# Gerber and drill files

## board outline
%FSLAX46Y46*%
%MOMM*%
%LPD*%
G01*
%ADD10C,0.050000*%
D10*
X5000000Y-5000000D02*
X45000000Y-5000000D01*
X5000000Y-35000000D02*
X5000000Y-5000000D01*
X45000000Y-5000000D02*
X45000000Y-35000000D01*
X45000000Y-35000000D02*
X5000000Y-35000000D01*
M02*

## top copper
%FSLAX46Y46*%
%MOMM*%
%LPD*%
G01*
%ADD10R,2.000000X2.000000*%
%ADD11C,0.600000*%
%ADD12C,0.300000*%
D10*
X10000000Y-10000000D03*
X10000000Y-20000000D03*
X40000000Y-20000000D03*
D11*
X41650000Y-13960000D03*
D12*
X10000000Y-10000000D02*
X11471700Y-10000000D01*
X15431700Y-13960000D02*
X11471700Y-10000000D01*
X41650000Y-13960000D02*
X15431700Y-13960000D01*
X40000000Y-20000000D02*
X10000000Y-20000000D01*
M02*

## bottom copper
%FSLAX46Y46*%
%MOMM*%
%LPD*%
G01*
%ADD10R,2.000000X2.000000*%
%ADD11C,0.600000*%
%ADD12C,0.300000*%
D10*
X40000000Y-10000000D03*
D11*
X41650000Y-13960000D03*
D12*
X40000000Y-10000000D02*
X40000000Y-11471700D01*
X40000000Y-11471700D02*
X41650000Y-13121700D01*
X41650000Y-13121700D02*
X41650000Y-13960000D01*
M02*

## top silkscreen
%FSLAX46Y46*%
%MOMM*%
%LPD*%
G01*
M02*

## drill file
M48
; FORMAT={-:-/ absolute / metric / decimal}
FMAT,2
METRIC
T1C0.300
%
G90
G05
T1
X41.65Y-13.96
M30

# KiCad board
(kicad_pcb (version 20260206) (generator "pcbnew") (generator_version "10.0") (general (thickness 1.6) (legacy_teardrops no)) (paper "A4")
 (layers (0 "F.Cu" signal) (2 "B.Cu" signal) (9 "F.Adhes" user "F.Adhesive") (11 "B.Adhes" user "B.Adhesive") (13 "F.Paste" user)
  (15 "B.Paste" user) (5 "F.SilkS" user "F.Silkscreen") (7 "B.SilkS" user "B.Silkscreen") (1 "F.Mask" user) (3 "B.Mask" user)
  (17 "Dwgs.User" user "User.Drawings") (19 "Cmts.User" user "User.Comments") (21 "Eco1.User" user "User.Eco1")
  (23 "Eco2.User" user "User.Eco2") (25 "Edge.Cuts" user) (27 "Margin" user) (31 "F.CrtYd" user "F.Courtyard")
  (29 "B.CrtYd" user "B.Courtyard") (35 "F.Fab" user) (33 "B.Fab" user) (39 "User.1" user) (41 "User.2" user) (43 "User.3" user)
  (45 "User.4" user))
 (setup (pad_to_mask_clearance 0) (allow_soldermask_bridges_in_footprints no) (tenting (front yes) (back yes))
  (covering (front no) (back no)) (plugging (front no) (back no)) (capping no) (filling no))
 (gr_line (start 5 5) (end 45 5) (stroke (width 0.05) (type default)) (layer "Edge.Cuts"))
 (gr_line (start 5 35) (end 5 5) (stroke (width 0.05) (type default)) (layer "Edge.Cuts"))
 (gr_line (start 45 5) (end 45 35) (stroke (width 0.05) (type default)) (layer "Edge.Cuts"))
 (gr_line (start 45 35) (end 5 35) (stroke (width 0.05) (type default)) (layer "Edge.Cuts"))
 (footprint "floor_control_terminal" (layer "F.Cu") (at 10 10)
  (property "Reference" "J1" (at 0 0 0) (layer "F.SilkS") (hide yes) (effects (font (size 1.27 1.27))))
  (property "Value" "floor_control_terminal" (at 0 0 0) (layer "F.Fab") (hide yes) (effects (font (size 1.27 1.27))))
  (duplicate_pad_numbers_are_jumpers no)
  (pad "1" smd rect (at 0 0) (size 2 2) (layers "F.Cu" "F.Paste" "F.Mask") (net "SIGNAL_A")))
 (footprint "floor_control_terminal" (layer "B.Cu") (at 40 10)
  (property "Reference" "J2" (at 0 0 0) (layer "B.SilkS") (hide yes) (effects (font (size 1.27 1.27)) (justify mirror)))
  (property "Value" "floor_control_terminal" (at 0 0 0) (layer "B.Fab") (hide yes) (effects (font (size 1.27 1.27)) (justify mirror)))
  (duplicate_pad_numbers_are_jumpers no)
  (pad "1" smd rect (at 0 0) (size 2 2) (layers "B.Cu" "B.Paste" "B.Mask") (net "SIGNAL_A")))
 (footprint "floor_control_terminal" (layer "F.Cu") (at 10 20)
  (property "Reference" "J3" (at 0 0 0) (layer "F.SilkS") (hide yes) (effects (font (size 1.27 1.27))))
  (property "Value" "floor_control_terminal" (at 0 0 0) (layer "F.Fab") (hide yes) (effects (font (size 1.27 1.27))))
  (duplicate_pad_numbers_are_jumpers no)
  (pad "1" smd rect (at 0 0) (size 2 2) (layers "F.Cu" "F.Paste" "F.Mask") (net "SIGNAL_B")))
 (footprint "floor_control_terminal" (layer "F.Cu") (at 40 20)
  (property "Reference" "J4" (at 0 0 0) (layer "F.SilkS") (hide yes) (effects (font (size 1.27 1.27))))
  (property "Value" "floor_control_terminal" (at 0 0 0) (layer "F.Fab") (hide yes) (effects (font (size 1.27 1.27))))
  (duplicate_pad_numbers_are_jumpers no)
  (pad "1" smd rect (at 0 0) (size 2 2) (layers "F.Cu" "F.Paste" "F.Mask") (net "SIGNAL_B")))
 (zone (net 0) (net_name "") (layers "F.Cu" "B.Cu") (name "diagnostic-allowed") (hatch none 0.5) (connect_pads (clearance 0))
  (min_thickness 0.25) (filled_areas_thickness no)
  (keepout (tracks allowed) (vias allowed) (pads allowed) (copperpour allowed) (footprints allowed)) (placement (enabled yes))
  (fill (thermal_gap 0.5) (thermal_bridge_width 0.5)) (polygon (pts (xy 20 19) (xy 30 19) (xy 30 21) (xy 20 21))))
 (segment (start 10 10) (end 11.4717 10) (width 0.3) (layer "F.Cu") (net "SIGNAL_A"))
 (segment (start 15.4317 13.96) (end 11.4717 10) (width 0.3) (layer "F.Cu") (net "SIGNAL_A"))
 (segment (start 41.65 13.96) (end 15.4317 13.96) (width 0.3) (layer "F.Cu") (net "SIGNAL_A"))
 (via (at 41.65 13.96) (size 0.6) (drill 0.3) (layers "F.Cu" "B.Cu") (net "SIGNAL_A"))
 (segment (start 40 10) (end 40 11.4717) (width 0.3) (layer "B.Cu") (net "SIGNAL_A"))
 (segment (start 40 11.4717) (end 41.65 13.1217) (width 0.3) (layer "B.Cu") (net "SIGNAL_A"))
 (segment (start 41.65 13.1217) (end 41.65 13.96) (width 0.3) (layer "B.Cu") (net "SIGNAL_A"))
 (segment (start 40 20) (end 10 20) (width 0.3) (layer "F.Cu") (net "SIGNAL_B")))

